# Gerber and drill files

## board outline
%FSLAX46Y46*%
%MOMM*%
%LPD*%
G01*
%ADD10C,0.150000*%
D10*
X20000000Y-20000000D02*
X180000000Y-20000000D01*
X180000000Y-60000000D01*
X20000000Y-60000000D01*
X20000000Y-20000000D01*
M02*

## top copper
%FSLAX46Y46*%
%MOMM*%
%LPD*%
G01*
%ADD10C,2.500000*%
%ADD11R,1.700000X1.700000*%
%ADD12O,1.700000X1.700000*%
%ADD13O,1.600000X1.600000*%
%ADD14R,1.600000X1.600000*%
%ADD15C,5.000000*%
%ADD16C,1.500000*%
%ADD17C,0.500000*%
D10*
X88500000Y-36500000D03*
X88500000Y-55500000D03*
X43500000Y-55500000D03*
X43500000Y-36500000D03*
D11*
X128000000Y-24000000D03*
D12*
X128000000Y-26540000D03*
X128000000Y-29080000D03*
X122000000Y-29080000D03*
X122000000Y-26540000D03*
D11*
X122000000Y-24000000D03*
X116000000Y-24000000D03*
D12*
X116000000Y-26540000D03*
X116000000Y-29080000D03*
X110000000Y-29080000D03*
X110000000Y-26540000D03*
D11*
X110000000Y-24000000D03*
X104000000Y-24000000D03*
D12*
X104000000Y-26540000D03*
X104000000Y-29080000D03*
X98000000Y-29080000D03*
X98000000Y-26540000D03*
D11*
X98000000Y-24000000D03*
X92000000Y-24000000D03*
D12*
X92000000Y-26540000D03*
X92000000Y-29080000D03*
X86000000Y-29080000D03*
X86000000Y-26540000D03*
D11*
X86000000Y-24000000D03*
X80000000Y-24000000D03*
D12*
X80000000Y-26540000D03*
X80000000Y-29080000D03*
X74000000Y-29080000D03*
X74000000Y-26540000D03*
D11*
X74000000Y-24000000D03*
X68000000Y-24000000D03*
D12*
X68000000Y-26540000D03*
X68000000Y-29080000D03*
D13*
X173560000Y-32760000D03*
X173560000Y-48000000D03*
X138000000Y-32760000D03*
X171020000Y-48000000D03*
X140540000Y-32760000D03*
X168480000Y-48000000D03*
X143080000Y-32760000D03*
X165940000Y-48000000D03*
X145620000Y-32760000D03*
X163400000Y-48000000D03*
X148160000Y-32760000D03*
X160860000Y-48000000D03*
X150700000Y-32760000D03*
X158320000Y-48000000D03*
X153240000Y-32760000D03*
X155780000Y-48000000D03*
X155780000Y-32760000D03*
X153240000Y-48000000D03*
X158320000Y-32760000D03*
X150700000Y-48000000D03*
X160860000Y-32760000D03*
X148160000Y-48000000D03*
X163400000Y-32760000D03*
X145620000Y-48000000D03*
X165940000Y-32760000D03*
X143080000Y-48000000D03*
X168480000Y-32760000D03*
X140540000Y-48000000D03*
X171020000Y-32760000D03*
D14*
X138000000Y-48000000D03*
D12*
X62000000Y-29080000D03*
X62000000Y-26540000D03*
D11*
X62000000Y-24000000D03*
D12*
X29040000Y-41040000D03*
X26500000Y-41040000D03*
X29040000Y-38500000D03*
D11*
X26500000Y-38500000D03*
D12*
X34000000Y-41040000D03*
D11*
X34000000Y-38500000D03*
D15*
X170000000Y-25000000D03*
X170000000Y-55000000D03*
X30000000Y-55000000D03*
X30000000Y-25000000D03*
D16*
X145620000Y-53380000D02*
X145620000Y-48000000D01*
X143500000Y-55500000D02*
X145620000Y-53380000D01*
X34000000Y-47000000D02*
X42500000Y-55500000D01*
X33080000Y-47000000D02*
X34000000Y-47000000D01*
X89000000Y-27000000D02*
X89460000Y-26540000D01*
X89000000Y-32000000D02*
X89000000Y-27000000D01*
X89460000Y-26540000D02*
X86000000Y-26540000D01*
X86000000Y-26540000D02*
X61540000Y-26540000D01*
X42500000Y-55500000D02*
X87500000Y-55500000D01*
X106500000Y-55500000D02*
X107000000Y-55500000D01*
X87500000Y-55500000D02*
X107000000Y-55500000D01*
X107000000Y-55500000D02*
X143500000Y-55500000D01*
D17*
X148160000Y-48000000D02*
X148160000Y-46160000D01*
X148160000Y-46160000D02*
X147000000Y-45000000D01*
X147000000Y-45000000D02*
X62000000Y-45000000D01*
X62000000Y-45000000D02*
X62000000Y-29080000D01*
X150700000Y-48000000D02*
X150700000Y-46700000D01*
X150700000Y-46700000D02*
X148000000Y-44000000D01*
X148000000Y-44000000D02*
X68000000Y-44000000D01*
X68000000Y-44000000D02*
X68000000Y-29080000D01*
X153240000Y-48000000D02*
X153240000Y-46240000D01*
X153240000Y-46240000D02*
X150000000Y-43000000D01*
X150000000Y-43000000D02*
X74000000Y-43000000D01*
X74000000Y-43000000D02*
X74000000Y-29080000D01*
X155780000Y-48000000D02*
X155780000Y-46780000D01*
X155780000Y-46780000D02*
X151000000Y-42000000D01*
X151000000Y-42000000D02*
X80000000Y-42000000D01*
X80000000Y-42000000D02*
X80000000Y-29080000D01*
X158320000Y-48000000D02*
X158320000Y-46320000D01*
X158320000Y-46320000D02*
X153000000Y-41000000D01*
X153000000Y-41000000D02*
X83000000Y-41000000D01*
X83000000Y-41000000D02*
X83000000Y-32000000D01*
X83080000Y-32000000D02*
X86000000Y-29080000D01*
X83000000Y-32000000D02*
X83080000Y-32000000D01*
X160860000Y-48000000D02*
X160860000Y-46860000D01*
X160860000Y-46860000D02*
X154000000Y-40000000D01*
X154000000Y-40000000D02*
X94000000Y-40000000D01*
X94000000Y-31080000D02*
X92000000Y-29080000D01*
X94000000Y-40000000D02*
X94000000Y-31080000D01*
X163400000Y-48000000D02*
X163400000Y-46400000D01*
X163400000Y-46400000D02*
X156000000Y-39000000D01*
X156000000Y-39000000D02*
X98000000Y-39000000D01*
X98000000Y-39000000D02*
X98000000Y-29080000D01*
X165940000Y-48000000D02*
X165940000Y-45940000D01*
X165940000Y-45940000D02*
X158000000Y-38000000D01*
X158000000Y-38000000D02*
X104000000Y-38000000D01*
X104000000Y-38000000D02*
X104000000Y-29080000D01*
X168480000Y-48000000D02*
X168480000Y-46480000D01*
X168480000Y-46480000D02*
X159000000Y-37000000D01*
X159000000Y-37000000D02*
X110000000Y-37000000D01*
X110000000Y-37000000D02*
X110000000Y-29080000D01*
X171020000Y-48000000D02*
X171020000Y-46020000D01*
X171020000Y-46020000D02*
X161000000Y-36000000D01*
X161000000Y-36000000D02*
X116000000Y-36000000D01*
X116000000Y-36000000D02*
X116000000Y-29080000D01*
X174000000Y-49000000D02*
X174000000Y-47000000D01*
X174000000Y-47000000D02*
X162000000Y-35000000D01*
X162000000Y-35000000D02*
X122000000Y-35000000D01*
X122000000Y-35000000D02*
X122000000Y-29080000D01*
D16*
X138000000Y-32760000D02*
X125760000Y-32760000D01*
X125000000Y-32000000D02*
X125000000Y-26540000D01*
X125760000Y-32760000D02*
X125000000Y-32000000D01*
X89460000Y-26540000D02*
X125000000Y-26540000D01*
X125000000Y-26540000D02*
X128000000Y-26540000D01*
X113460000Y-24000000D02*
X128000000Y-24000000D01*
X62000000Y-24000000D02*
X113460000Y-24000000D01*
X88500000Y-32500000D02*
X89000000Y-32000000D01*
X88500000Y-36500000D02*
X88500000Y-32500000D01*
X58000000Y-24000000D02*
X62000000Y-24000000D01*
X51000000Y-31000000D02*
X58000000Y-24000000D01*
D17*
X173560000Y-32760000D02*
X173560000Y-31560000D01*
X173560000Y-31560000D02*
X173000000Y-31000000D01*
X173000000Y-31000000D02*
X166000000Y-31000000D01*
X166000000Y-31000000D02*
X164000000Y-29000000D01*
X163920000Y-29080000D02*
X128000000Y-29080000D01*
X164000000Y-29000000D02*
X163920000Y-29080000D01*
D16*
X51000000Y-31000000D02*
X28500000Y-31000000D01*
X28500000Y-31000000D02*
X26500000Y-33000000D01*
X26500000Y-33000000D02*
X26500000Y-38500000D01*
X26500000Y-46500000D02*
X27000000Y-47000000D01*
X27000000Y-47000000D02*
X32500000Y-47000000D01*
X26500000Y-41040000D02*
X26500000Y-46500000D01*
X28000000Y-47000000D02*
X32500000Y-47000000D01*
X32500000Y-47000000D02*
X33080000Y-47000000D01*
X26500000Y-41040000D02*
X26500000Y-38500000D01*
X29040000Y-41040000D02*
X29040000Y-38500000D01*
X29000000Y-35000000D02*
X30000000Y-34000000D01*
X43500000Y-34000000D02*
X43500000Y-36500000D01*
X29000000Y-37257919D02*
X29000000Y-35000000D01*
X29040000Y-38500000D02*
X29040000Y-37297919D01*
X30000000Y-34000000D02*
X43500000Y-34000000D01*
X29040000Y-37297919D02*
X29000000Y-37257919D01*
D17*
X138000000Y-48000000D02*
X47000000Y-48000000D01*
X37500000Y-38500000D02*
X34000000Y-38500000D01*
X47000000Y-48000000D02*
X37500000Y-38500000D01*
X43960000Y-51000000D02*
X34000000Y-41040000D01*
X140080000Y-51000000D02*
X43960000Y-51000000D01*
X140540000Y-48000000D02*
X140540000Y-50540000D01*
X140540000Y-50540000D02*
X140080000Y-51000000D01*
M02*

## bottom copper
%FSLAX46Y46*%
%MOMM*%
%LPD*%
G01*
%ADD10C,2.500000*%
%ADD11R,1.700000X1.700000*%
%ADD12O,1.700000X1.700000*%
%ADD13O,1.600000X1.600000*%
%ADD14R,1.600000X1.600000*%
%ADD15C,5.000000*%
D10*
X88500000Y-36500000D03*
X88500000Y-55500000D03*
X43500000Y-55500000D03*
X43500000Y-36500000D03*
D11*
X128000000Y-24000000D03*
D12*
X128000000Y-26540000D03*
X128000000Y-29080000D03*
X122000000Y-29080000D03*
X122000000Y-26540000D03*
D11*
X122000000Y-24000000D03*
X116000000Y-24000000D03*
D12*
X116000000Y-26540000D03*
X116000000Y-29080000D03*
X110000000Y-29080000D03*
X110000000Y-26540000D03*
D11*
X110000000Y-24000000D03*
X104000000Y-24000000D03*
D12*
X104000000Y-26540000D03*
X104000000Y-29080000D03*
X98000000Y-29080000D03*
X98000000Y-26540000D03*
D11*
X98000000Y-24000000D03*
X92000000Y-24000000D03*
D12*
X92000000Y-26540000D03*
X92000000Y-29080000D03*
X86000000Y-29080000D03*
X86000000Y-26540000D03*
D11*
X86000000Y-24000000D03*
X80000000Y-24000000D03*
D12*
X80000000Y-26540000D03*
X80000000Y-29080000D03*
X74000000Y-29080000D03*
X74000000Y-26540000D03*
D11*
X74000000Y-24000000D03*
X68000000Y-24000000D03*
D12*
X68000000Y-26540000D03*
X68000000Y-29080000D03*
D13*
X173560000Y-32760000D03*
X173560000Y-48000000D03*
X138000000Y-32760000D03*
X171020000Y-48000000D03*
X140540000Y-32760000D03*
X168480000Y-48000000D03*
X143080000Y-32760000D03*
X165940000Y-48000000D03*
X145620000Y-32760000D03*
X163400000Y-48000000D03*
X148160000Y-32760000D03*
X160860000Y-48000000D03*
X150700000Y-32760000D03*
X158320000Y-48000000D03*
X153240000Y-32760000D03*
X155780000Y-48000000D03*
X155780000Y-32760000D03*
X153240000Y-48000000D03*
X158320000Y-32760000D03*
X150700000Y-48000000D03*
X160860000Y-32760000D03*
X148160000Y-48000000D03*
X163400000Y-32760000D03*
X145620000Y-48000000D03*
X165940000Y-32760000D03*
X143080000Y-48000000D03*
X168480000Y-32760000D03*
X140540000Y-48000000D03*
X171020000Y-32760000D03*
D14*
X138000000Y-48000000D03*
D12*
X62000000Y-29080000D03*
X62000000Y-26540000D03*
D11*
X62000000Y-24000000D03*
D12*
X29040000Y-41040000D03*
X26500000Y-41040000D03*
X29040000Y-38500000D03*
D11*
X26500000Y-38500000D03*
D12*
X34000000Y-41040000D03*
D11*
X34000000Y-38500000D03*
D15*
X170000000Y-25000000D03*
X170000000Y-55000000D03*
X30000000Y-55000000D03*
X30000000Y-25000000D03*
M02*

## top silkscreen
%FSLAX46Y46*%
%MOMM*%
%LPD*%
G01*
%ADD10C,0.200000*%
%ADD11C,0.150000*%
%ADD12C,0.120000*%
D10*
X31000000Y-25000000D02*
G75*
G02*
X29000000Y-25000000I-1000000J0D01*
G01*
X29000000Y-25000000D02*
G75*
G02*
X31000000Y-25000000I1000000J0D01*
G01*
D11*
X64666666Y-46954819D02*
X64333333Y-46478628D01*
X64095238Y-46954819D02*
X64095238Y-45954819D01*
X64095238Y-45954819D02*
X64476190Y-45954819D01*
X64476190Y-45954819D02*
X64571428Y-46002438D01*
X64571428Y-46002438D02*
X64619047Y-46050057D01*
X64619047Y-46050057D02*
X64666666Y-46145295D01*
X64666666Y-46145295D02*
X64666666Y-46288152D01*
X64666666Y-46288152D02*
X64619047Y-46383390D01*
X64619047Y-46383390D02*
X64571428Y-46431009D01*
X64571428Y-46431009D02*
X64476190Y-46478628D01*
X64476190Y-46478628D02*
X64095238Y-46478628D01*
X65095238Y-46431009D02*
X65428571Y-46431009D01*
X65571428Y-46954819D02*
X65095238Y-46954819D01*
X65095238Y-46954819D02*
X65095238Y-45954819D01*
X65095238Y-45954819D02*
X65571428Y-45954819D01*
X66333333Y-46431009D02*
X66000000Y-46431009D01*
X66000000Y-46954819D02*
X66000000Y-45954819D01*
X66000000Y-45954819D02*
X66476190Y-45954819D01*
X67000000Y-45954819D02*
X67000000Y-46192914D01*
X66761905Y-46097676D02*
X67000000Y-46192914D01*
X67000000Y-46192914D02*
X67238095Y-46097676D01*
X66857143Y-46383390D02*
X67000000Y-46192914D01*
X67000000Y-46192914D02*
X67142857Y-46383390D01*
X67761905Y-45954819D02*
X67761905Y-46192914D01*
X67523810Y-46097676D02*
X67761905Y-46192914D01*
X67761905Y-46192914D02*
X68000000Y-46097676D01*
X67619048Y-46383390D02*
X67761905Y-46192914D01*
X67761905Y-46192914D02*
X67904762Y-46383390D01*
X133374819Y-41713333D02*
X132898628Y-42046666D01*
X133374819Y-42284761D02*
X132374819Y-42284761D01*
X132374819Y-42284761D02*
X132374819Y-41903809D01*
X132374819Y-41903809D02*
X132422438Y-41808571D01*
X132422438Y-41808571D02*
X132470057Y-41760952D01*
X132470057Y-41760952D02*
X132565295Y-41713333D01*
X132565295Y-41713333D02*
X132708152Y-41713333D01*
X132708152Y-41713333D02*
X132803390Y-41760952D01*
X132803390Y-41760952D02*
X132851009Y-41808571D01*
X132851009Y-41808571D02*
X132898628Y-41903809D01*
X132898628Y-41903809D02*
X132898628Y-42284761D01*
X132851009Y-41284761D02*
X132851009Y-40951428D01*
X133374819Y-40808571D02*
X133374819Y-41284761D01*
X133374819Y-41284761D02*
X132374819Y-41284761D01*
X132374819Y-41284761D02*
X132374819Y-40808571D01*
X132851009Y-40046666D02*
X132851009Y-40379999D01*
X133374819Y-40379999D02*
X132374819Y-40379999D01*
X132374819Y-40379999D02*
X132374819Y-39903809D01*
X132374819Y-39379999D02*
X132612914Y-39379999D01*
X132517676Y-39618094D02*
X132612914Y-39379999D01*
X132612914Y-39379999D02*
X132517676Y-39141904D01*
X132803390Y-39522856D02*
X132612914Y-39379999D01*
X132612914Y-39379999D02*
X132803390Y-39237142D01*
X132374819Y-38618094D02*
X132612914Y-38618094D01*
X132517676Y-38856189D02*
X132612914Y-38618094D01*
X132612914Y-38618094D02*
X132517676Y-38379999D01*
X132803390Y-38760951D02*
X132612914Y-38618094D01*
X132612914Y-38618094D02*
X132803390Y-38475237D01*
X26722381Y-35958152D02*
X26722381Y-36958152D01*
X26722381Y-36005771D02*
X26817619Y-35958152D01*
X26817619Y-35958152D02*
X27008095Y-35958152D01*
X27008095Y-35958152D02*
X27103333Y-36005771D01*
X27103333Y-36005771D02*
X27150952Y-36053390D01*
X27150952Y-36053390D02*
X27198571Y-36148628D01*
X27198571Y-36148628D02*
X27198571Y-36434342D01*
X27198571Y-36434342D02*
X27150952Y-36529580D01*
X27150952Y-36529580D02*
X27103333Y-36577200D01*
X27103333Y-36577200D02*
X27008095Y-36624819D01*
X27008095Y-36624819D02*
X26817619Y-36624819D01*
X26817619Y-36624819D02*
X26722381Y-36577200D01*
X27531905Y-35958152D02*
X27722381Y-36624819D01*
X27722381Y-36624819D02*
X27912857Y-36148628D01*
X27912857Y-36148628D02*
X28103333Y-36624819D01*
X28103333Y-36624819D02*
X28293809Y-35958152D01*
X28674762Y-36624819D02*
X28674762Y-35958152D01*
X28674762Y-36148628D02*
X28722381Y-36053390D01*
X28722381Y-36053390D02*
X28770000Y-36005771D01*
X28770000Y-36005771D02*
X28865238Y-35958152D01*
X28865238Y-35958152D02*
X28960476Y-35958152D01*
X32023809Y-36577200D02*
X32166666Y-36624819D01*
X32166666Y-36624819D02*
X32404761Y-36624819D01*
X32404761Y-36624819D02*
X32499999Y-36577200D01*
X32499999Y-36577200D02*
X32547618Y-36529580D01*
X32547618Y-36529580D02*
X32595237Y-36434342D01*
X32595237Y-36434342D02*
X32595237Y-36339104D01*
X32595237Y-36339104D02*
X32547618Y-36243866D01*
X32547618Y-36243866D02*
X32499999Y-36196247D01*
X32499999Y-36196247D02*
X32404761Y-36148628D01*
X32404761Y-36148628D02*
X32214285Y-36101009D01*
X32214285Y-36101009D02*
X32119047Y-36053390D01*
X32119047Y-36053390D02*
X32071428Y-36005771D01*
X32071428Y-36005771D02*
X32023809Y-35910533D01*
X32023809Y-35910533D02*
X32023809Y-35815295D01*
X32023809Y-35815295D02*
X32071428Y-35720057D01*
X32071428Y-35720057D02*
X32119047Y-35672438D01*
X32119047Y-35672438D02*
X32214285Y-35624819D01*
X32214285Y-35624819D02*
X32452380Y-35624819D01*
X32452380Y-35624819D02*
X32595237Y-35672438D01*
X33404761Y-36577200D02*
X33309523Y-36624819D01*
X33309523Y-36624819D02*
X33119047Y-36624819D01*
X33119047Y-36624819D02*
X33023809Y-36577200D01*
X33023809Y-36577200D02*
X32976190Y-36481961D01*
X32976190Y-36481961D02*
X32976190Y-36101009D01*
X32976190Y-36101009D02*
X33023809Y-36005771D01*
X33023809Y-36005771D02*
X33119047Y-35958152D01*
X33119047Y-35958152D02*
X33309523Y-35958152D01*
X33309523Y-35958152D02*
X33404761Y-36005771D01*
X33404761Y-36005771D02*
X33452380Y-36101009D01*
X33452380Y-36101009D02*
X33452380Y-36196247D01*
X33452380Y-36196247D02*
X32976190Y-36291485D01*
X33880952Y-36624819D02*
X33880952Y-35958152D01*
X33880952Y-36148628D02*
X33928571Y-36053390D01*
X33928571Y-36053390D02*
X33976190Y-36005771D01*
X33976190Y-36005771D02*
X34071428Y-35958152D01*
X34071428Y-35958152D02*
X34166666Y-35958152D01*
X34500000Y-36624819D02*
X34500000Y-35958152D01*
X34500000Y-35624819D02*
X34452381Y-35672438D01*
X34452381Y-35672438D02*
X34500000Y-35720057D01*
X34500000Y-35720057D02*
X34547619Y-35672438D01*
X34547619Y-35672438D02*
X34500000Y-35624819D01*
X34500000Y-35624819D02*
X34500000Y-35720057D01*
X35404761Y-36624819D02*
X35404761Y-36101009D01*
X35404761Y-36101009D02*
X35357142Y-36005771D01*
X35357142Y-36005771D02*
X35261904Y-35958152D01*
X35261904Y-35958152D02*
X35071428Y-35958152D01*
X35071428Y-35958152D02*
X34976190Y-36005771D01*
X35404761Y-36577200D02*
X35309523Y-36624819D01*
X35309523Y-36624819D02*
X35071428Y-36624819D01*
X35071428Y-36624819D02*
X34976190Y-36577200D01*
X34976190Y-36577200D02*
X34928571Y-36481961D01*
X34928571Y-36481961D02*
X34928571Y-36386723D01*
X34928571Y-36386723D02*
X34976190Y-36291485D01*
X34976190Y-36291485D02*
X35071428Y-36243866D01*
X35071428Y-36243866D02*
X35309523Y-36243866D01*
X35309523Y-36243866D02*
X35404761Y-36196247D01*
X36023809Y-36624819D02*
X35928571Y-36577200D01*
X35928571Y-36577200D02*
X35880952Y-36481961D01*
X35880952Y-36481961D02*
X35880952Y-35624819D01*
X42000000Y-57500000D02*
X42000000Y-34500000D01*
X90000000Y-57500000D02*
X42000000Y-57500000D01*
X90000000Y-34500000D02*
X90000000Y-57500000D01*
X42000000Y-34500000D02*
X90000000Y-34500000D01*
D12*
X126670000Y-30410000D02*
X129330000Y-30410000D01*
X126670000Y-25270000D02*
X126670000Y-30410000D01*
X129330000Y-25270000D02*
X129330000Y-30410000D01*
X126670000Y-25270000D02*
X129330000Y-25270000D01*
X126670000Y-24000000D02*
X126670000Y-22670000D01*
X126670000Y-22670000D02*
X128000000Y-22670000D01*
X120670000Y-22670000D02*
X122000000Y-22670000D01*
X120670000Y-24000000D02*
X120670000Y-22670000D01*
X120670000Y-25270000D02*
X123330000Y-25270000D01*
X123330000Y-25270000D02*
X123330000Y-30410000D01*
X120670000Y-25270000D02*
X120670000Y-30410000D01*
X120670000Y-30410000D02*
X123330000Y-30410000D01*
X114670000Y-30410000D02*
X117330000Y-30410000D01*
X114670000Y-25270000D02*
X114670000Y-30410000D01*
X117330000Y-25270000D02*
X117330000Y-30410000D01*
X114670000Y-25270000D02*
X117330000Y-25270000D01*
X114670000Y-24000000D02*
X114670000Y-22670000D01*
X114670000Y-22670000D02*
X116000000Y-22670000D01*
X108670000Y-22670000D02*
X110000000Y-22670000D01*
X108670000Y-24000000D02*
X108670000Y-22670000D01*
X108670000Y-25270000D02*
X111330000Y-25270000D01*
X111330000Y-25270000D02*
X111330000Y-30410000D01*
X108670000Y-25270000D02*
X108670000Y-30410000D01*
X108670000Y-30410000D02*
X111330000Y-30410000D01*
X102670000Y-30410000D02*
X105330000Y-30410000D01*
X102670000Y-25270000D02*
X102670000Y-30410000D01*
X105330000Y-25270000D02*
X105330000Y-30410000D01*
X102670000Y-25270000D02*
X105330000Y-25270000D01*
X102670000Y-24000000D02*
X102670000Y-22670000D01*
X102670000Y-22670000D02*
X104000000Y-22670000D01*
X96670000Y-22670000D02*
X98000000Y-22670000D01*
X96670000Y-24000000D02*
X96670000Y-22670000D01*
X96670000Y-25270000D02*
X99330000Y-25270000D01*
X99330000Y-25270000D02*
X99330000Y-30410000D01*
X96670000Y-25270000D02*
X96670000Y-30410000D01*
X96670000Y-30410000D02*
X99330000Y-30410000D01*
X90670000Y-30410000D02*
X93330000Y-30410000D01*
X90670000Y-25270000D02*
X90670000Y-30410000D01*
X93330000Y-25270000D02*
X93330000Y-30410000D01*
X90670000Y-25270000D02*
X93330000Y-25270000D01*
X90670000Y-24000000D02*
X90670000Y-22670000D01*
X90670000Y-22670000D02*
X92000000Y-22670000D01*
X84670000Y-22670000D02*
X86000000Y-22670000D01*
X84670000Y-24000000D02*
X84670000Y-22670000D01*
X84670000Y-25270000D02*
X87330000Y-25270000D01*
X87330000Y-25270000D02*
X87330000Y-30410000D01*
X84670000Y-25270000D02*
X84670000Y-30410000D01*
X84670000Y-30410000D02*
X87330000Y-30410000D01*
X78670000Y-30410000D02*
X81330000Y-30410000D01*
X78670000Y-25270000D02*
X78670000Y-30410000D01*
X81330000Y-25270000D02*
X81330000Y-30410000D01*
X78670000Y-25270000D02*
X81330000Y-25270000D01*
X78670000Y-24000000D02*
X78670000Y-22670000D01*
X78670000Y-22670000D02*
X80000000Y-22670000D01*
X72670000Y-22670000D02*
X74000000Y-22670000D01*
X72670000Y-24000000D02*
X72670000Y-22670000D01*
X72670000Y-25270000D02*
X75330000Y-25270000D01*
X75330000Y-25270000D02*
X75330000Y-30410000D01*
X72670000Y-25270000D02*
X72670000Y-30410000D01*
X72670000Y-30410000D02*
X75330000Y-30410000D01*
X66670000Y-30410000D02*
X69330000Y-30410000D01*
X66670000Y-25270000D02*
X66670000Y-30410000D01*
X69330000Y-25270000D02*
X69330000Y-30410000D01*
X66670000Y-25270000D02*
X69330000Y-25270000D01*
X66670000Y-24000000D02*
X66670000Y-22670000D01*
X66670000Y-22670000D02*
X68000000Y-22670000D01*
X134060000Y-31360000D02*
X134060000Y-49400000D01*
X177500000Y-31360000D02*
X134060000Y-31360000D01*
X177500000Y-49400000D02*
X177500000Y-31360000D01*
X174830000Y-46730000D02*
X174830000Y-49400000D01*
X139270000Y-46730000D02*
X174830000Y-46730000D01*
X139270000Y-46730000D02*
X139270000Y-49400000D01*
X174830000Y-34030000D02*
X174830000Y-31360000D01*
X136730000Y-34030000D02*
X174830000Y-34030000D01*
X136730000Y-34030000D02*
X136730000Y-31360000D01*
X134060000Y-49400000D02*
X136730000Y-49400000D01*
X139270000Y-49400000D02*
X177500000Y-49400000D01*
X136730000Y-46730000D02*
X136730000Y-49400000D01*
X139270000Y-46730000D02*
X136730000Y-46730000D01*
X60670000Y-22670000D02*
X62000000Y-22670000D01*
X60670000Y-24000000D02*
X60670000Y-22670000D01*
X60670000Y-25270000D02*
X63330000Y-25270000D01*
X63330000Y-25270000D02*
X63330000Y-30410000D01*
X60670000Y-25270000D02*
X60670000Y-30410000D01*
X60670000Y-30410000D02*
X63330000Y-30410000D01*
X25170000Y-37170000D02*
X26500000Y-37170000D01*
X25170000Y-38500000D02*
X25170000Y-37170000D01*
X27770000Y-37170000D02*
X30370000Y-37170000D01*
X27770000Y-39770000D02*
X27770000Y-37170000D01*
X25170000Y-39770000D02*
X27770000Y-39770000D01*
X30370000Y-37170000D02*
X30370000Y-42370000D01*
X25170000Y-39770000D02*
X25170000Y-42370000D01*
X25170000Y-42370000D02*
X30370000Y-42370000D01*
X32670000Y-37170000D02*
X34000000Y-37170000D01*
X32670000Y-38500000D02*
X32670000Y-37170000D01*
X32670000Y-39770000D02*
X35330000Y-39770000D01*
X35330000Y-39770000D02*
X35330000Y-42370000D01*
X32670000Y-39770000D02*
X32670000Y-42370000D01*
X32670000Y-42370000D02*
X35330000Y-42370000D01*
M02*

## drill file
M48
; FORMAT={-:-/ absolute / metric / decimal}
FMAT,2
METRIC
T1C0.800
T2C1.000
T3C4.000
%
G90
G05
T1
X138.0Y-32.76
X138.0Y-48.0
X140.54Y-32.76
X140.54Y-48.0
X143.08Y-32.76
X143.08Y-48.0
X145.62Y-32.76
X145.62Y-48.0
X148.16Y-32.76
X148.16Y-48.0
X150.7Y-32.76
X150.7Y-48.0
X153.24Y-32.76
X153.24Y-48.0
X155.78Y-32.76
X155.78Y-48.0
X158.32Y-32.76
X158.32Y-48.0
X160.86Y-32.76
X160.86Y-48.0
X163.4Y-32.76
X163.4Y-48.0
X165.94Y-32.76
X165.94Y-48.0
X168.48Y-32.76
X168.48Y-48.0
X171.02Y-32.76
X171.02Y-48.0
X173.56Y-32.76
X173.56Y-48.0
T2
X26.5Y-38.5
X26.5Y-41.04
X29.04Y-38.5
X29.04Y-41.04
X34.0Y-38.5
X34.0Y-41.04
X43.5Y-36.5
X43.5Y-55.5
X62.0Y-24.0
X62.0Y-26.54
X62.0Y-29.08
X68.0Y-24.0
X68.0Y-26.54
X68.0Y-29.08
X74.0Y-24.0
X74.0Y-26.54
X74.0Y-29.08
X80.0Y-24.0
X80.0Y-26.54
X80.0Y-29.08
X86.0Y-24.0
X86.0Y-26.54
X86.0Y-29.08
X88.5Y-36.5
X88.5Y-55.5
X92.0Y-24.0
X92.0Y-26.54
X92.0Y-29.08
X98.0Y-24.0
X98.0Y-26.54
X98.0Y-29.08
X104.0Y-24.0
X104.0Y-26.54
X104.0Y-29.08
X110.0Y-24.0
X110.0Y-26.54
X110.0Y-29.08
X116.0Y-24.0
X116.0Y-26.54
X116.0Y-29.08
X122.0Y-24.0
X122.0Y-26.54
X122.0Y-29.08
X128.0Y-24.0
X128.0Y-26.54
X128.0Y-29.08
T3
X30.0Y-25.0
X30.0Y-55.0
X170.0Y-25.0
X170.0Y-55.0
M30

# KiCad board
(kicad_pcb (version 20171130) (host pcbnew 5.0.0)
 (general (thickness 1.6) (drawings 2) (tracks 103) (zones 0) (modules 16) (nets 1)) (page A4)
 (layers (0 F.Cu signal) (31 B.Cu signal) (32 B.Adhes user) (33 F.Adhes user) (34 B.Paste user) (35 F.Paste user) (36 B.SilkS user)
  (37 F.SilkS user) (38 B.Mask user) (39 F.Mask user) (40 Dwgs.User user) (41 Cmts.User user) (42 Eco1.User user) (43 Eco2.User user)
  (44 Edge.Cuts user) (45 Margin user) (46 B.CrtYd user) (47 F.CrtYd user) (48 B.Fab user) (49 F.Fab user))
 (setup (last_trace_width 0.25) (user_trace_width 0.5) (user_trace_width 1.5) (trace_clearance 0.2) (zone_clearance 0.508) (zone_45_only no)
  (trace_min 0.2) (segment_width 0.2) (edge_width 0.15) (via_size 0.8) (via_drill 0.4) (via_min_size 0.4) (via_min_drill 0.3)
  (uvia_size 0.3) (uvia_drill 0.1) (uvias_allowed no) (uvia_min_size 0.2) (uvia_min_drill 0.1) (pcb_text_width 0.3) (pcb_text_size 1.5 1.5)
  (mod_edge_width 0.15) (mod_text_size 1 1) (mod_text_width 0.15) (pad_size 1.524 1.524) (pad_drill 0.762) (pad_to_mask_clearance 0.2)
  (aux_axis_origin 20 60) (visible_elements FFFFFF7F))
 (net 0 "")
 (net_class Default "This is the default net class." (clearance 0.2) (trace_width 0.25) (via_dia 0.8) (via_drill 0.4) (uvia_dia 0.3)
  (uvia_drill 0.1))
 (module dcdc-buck (layer F.Cu) (at 66 46)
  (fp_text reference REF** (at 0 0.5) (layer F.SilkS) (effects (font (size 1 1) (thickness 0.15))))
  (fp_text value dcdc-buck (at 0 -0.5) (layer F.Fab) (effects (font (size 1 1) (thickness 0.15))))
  (fp_line (start -24 11.5) (end -24 -11.5) (layer F.SilkS) (width 0.15))
  (fp_line (start 24 11.5) (end -24 11.5) (layer F.SilkS) (width 0.15))
  (fp_line (start 24 -11.5) (end 24 11.5) (layer F.SilkS) (width 0.15))
  (fp_line (start -24 -11.5) (end 24 -11.5) (layer F.SilkS) (width 0.15))
  (pad 4 thru_hole circle (at 22.5 -9.5) (size 2.5 2.5) (drill 1) (layers *.Cu *.Mask))
  (pad 3 thru_hole circle (at 22.5 9.5) (size 2.5 2.5) (drill 1) (layers *.Cu *.Mask))
  (pad 2 thru_hole circle (at -22.5 9.5) (size 2.5 2.5) (drill 1) (layers *.Cu *.Mask))
  (pad 1 thru_hole circle (at -22.5 -9.5) (size 2.5 2.5) (drill 1) (layers *.Cu *.Mask)))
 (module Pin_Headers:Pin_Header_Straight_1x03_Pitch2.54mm (layer F.Cu) (at 128 24)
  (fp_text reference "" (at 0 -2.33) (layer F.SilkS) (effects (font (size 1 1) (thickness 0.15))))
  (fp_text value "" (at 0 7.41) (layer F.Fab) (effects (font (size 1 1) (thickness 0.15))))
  (fp_line (start -1.33 6.41) (end 1.33 6.41) (layer F.SilkS) (width 0.12))
  (fp_line (start -1.33 1.27) (end -1.33 6.41) (layer F.SilkS) (width 0.12))
  (fp_line (start 1.33 1.27) (end 1.33 6.41) (layer F.SilkS) (width 0.12))
  (fp_line (start -1.33 1.27) (end 1.33 1.27) (layer F.SilkS) (width 0.12))
  (fp_line (start -1.33 0) (end -1.33 -1.33) (layer F.SilkS) (width 0.12))
  (fp_line (start -1.33 -1.33) (end 0 -1.33) (layer F.SilkS) (width 0.12))
  (pad 1 thru_hole rect (at 0 0) (size 1.7 1.7) (drill 1) (layers *.Cu *.Mask))
  (pad 2 thru_hole oval (at 0 2.54) (size 1.7 1.7) (drill 1) (layers *.Cu *.Mask))
  (pad 3 thru_hole oval (at 0 5.08) (size 1.7 1.7) (drill 1) (layers *.Cu *.Mask)))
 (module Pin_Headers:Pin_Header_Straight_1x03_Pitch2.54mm (layer F.Cu) (at 122 24)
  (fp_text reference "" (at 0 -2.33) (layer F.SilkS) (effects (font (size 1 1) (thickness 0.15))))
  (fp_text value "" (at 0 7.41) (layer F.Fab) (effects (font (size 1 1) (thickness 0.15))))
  (fp_line (start -1.33 -1.33) (end 0 -1.33) (layer F.SilkS) (width 0.12))
  (fp_line (start -1.33 0) (end -1.33 -1.33) (layer F.SilkS) (width 0.12))
  (fp_line (start -1.33 1.27) (end 1.33 1.27) (layer F.SilkS) (width 0.12))
  (fp_line (start 1.33 1.27) (end 1.33 6.41) (layer F.SilkS) (width 0.12))
  (fp_line (start -1.33 1.27) (end -1.33 6.41) (layer F.SilkS) (width 0.12))
  (fp_line (start -1.33 6.41) (end 1.33 6.41) (layer F.SilkS) (width 0.12))
  (pad 3 thru_hole oval (at 0 5.08) (size 1.7 1.7) (drill 1) (layers *.Cu *.Mask))
  (pad 2 thru_hole oval (at 0 2.54) (size 1.7 1.7) (drill 1) (layers *.Cu *.Mask))
  (pad 1 thru_hole rect (at 0 0) (size 1.7 1.7) (drill 1) (layers *.Cu *.Mask)))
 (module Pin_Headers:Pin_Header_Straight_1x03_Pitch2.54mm (layer F.Cu) (at 116 24)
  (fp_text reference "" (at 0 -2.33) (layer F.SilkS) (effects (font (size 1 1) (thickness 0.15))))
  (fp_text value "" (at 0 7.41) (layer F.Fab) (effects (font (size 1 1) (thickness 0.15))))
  (fp_line (start -1.33 6.41) (end 1.33 6.41) (layer F.SilkS) (width 0.12))
  (fp_line (start -1.33 1.27) (end -1.33 6.41) (layer F.SilkS) (width 0.12))
  (fp_line (start 1.33 1.27) (end 1.33 6.41) (layer F.SilkS) (width 0.12))
  (fp_line (start -1.33 1.27) (end 1.33 1.27) (layer F.SilkS) (width 0.12))
  (fp_line (start -1.33 0) (end -1.33 -1.33) (layer F.SilkS) (width 0.12))
  (fp_line (start -1.33 -1.33) (end 0 -1.33) (layer F.SilkS) (width 0.12))
  (pad 1 thru_hole rect (at 0 0) (size 1.7 1.7) (drill 1) (layers *.Cu *.Mask))
  (pad 2 thru_hole oval (at 0 2.54) (size 1.7 1.7) (drill 1) (layers *.Cu *.Mask))
  (pad 3 thru_hole oval (at 0 5.08) (size 1.7 1.7) (drill 1) (layers *.Cu *.Mask)))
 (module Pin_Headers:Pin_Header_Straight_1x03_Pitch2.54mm (layer F.Cu) (at 110 24)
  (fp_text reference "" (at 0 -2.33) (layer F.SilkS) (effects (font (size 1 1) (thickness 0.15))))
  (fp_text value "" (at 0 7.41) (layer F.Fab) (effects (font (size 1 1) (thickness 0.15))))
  (fp_line (start -1.33 -1.33) (end 0 -1.33) (layer F.SilkS) (width 0.12))
  (fp_line (start -1.33 0) (end -1.33 -1.33) (layer F.SilkS) (width 0.12))
  (fp_line (start -1.33 1.27) (end 1.33 1.27) (layer F.SilkS) (width 0.12))
  (fp_line (start 1.33 1.27) (end 1.33 6.41) (layer F.SilkS) (width 0.12))
  (fp_line (start -1.33 1.27) (end -1.33 6.41) (layer F.SilkS) (width 0.12))
  (fp_line (start -1.33 6.41) (end 1.33 6.41) (layer F.SilkS) (width 0.12))
  (pad 3 thru_hole oval (at 0 5.08) (size 1.7 1.7) (drill 1) (layers *.Cu *.Mask))
  (pad 2 thru_hole oval (at 0 2.54) (size 1.7 1.7) (drill 1) (layers *.Cu *.Mask))
  (pad 1 thru_hole rect (at 0 0) (size 1.7 1.7) (drill 1) (layers *.Cu *.Mask)))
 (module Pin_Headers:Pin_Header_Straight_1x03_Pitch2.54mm (layer F.Cu) (at 104 24)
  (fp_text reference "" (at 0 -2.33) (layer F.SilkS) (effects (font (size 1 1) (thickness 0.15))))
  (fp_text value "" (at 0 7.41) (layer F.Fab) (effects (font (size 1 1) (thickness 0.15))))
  (fp_line (start -1.33 6.41) (end 1.33 6.41) (layer F.SilkS) (width 0.12))
  (fp_line (start -1.33 1.27) (end -1.33 6.41) (layer F.SilkS) (width 0.12))
  (fp_line (start 1.33 1.27) (end 1.33 6.41) (layer F.SilkS) (width 0.12))
  (fp_line (start -1.33 1.27) (end 1.33 1.27) (layer F.SilkS) (width 0.12))
  (fp_line (start -1.33 0) (end -1.33 -1.33) (layer F.SilkS) (width 0.12))
  (fp_line (start -1.33 -1.33) (end 0 -1.33) (layer F.SilkS) (width 0.12))
  (pad 1 thru_hole rect (at 0 0) (size 1.7 1.7) (drill 1) (layers *.Cu *.Mask))
  (pad 2 thru_hole oval (at 0 2.54) (size 1.7 1.7) (drill 1) (layers *.Cu *.Mask))
  (pad 3 thru_hole oval (at 0 5.08) (size 1.7 1.7) (drill 1) (layers *.Cu *.Mask)))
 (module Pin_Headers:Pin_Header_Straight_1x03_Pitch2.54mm (layer F.Cu) (at 98 24)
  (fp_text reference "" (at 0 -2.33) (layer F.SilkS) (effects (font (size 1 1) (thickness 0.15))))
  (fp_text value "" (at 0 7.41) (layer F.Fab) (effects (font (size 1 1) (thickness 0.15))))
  (fp_line (start -1.33 -1.33) (end 0 -1.33) (layer F.SilkS) (width 0.12))
  (fp_line (start -1.33 0) (end -1.33 -1.33) (layer F.SilkS) (width 0.12))
  (fp_line (start -1.33 1.27) (end 1.33 1.27) (layer F.SilkS) (width 0.12))
  (fp_line (start 1.33 1.27) (end 1.33 6.41) (layer F.SilkS) (width 0.12))
  (fp_line (start -1.33 1.27) (end -1.33 6.41) (layer F.SilkS) (width 0.12))
  (fp_line (start -1.33 6.41) (end 1.33 6.41) (layer F.SilkS) (width 0.12))
  (pad 3 thru_hole oval (at 0 5.08) (size 1.7 1.7) (drill 1) (layers *.Cu *.Mask))
  (pad 2 thru_hole oval (at 0 2.54) (size 1.7 1.7) (drill 1) (layers *.Cu *.Mask))
  (pad 1 thru_hole rect (at 0 0) (size 1.7 1.7) (drill 1) (layers *.Cu *.Mask)))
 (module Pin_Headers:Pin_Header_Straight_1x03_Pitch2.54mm (layer F.Cu) (at 92 24)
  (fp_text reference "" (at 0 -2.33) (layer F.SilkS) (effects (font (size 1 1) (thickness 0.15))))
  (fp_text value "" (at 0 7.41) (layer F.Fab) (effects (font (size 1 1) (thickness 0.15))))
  (fp_line (start -1.33 6.41) (end 1.33 6.41) (layer F.SilkS) (width 0.12))
  (fp_line (start -1.33 1.27) (end -1.33 6.41) (layer F.SilkS) (width 0.12))
  (fp_line (start 1.33 1.27) (end 1.33 6.41) (layer F.SilkS) (width 0.12))
  (fp_line (start -1.33 1.27) (end 1.33 1.27) (layer F.SilkS) (width 0.12))
  (fp_line (start -1.33 0) (end -1.33 -1.33) (layer F.SilkS) (width 0.12))
  (fp_line (start -1.33 -1.33) (end 0 -1.33) (layer F.SilkS) (width 0.12))
  (pad 1 thru_hole rect (at 0 0) (size 1.7 1.7) (drill 1) (layers *.Cu *.Mask))
  (pad 2 thru_hole oval (at 0 2.54) (size 1.7 1.7) (drill 1) (layers *.Cu *.Mask))
  (pad 3 thru_hole oval (at 0 5.08) (size 1.7 1.7) (drill 1) (layers *.Cu *.Mask)))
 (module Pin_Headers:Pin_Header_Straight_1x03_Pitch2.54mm (layer F.Cu) (at 86 24)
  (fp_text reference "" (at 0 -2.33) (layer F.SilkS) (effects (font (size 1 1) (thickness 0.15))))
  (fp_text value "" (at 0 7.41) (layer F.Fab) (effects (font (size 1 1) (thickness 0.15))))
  (fp_line (start -1.33 -1.33) (end 0 -1.33) (layer F.SilkS) (width 0.12))
  (fp_line (start -1.33 0) (end -1.33 -1.33) (layer F.SilkS) (width 0.12))
  (fp_line (start -1.33 1.27) (end 1.33 1.27) (layer F.SilkS) (width 0.12))
  (fp_line (start 1.33 1.27) (end 1.33 6.41) (layer F.SilkS) (width 0.12))
  (fp_line (start -1.33 1.27) (end -1.33 6.41) (layer F.SilkS) (width 0.12))
  (fp_line (start -1.33 6.41) (end 1.33 6.41) (layer F.SilkS) (width 0.12))
  (pad 3 thru_hole oval (at 0 5.08) (size 1.7 1.7) (drill 1) (layers *.Cu *.Mask))
  (pad 2 thru_hole oval (at 0 2.54) (size 1.7 1.7) (drill 1) (layers *.Cu *.Mask))
  (pad 1 thru_hole rect (at 0 0) (size 1.7 1.7) (drill 1) (layers *.Cu *.Mask)))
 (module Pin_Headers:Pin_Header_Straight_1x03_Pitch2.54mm (layer F.Cu) (at 80 24)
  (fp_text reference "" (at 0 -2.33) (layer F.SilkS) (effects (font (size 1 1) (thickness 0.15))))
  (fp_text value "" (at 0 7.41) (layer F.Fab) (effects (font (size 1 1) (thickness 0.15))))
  (fp_line (start -1.33 6.41) (end 1.33 6.41) (layer F.SilkS) (width 0.12))
  (fp_line (start -1.33 1.27) (end -1.33 6.41) (layer F.SilkS) (width 0.12))
  (fp_line (start 1.33 1.27) (end 1.33 6.41) (layer F.SilkS) (width 0.12))
  (fp_line (start -1.33 1.27) (end 1.33 1.27) (layer F.SilkS) (width 0.12))
  (fp_line (start -1.33 0) (end -1.33 -1.33) (layer F.SilkS) (width 0.12))
  (fp_line (start -1.33 -1.33) (end 0 -1.33) (layer F.SilkS) (width 0.12))
  (pad 1 thru_hole rect (at 0 0) (size 1.7 1.7) (drill 1) (layers *.Cu *.Mask))
  (pad 2 thru_hole oval (at 0 2.54) (size 1.7 1.7) (drill 1) (layers *.Cu *.Mask))
  (pad 3 thru_hole oval (at 0 5.08) (size 1.7 1.7) (drill 1) (layers *.Cu *.Mask)))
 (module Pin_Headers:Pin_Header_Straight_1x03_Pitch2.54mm (layer F.Cu) (at 74 24)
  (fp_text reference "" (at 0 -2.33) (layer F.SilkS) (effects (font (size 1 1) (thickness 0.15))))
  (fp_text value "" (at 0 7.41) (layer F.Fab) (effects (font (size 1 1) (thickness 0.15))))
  (fp_line (start -1.33 -1.33) (end 0 -1.33) (layer F.SilkS) (width 0.12))
  (fp_line (start -1.33 0) (end -1.33 -1.33) (layer F.SilkS) (width 0.12))
  (fp_line (start -1.33 1.27) (end 1.33 1.27) (layer F.SilkS) (width 0.12))
  (fp_line (start 1.33 1.27) (end 1.33 6.41) (layer F.SilkS) (width 0.12))
  (fp_line (start -1.33 1.27) (end -1.33 6.41) (layer F.SilkS) (width 0.12))
  (fp_line (start -1.33 6.41) (end 1.33 6.41) (layer F.SilkS) (width 0.12))
  (pad 3 thru_hole oval (at 0 5.08) (size 1.7 1.7) (drill 1) (layers *.Cu *.Mask))
  (pad 2 thru_hole oval (at 0 2.54) (size 1.7 1.7) (drill 1) (layers *.Cu *.Mask))
  (pad 1 thru_hole rect (at 0 0) (size 1.7 1.7) (drill 1) (layers *.Cu *.Mask)))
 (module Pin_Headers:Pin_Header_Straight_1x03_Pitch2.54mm (layer F.Cu) (at 68 24)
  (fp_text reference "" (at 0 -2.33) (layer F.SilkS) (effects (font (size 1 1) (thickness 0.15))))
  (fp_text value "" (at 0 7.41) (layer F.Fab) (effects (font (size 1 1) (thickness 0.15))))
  (fp_line (start -1.33 6.41) (end 1.33 6.41) (layer F.SilkS) (width 0.12))
  (fp_line (start -1.33 1.27) (end -1.33 6.41) (layer F.SilkS) (width 0.12))
  (fp_line (start 1.33 1.27) (end 1.33 6.41) (layer F.SilkS) (width 0.12))
  (fp_line (start -1.33 1.27) (end 1.33 1.27) (layer F.SilkS) (width 0.12))
  (fp_line (start -1.33 0) (end -1.33 -1.33) (layer F.SilkS) (width 0.12))
  (fp_line (start -1.33 -1.33) (end 0 -1.33) (layer F.SilkS) (width 0.12))
  (pad 1 thru_hole rect (at 0 0) (size 1.7 1.7) (drill 1) (layers *.Cu *.Mask))
  (pad 2 thru_hole oval (at 0 2.54) (size 1.7 1.7) (drill 1) (layers *.Cu *.Mask))
  (pad 3 thru_hole oval (at 0 5.08) (size 1.7 1.7) (drill 1) (layers *.Cu *.Mask)))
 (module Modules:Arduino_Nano (layer F.Cu) (at 138 48 90)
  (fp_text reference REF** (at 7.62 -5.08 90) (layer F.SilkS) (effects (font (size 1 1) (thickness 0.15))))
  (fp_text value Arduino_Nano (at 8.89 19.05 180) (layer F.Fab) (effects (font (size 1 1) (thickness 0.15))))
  (fp_line (start 16.64 -3.94) (end -1.4 -3.94) (layer F.SilkS) (width 0.12))
  (fp_line (start 16.64 39.5) (end 16.64 -3.94) (layer F.SilkS) (width 0.12))
  (fp_line (start -1.4 39.5) (end 16.64 39.5) (layer F.SilkS) (width 0.12))
  (fp_line (start 1.27 36.83) (end -1.4 36.83) (layer F.SilkS) (width 0.12))
  (fp_line (start 1.27 1.27) (end 1.27 36.83) (layer F.SilkS) (width 0.12))
  (fp_line (start 1.27 1.27) (end -1.4 1.27) (layer F.SilkS) (width 0.12))
  (fp_line (start 13.97 36.83) (end 16.64 36.83) (layer F.SilkS) (width 0.12))
  (fp_line (start 13.97 -1.27) (end 13.97 36.83) (layer F.SilkS) (width 0.12))
  (fp_line (start 13.97 -1.27) (end 16.64 -1.27) (layer F.SilkS) (width 0.12))
  (fp_line (start -1.4 -3.94) (end -1.4 -1.27) (layer F.SilkS) (width 0.12))
  (fp_line (start -1.4 1.27) (end -1.4 39.5) (layer F.SilkS) (width 0.12))
  (fp_line (start 1.27 -1.27) (end -1.4 -1.27) (layer F.SilkS) (width 0.12))
  (fp_line (start 1.27 1.27) (end 1.27 -1.27) (layer F.SilkS) (width 0.12))
  (pad 16 thru_hole oval (at 15.24 35.56 90) (size 1.6 1.6) (drill 0.8) (layers *.Cu *.Mask))
  (pad 15 thru_hole oval (at 0 35.56 90) (size 1.6 1.6) (drill 0.8) (layers *.Cu *.Mask))
  (pad 30 thru_hole oval (at 15.24 0 90) (size 1.6 1.6) (drill 0.8) (layers *.Cu *.Mask))
  (pad 14 thru_hole oval (at 0 33.02 90) (size 1.6 1.6) (drill 0.8) (layers *.Cu *.Mask))
  (pad 29 thru_hole oval (at 15.24 2.54 90) (size 1.6 1.6) (drill 0.8) (layers *.Cu *.Mask))
  (pad 13 thru_hole oval (at 0 30.48 90) (size 1.6 1.6) (drill 0.8) (layers *.Cu *.Mask))
  (pad 28 thru_hole oval (at 15.24 5.08 90) (size 1.6 1.6) (drill 0.8) (layers *.Cu *.Mask))
  (pad 12 thru_hole oval (at 0 27.94 90) (size 1.6 1.6) (drill 0.8) (layers *.Cu *.Mask))
  (pad 27 thru_hole oval (at 15.24 7.62 90) (size 1.6 1.6) (drill 0.8) (layers *.Cu *.Mask))
  (pad 11 thru_hole oval (at 0 25.4 90) (size 1.6 1.6) (drill 0.8) (layers *.Cu *.Mask))
  (pad 26 thru_hole oval (at 15.24 10.16 90) (size 1.6 1.6) (drill 0.8) (layers *.Cu *.Mask))
  (pad 10 thru_hole oval (at 0 22.86 90) (size 1.6 1.6) (drill 0.8) (layers *.Cu *.Mask))
  (pad 25 thru_hole oval (at 15.24 12.7 90) (size 1.6 1.6) (drill 0.8) (layers *.Cu *.Mask))
  (pad 9 thru_hole oval (at 0 20.32 90) (size 1.6 1.6) (drill 0.8) (layers *.Cu *.Mask))
  (pad 24 thru_hole oval (at 15.24 15.24 90) (size 1.6 1.6) (drill 0.8) (layers *.Cu *.Mask))
  (pad 8 thru_hole oval (at 0 17.78 90) (size 1.6 1.6) (drill 0.8) (layers *.Cu *.Mask))
  (pad 23 thru_hole oval (at 15.24 17.78 90) (size 1.6 1.6) (drill 0.8) (layers *.Cu *.Mask))
  (pad 7 thru_hole oval (at 0 15.24 90) (size 1.6 1.6) (drill 0.8) (layers *.Cu *.Mask))
  (pad 22 thru_hole oval (at 15.24 20.32 90) (size 1.6 1.6) (drill 0.8) (layers *.Cu *.Mask))
  (pad 6 thru_hole oval (at 0 12.7 90) (size 1.6 1.6) (drill 0.8) (layers *.Cu *.Mask))
  (pad 21 thru_hole oval (at 15.24 22.86 90) (size 1.6 1.6) (drill 0.8) (layers *.Cu *.Mask))
  (pad 5 thru_hole oval (at 0 10.16 90) (size 1.6 1.6) (drill 0.8) (layers *.Cu *.Mask))
  (pad 20 thru_hole oval (at 15.24 25.4 90) (size 1.6 1.6) (drill 0.8) (layers *.Cu *.Mask))
  (pad 4 thru_hole oval (at 0 7.62 90) (size 1.6 1.6) (drill 0.8) (layers *.Cu *.Mask))
  (pad 19 thru_hole oval (at 15.24 27.94 90) (size 1.6 1.6) (drill 0.8) (layers *.Cu *.Mask))
  (pad 3 thru_hole oval (at 0 5.08 90) (size 1.6 1.6) (drill 0.8) (layers *.Cu *.Mask))
  (pad 18 thru_hole oval (at 15.24 30.48 90) (size 1.6 1.6) (drill 0.8) (layers *.Cu *.Mask))
  (pad 2 thru_hole oval (at 0 2.54 90) (size 1.6 1.6) (drill 0.8) (layers *.Cu *.Mask))
  (pad 17 thru_hole oval (at 15.24 33.02 90) (size 1.6 1.6) (drill 0.8) (layers *.Cu *.Mask))
  (pad 1 thru_hole rect (at 0 0 90) (size 1.6 1.6) (drill 0.8) (layers *.Cu *.Mask)))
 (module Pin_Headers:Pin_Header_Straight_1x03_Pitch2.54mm (layer F.Cu) (at 62 24)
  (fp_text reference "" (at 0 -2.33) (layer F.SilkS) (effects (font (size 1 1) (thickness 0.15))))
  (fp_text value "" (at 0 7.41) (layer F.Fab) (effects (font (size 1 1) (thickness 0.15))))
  (fp_line (start -1.33 -1.33) (end 0 -1.33) (layer F.SilkS) (width 0.12))
  (fp_line (start -1.33 0) (end -1.33 -1.33) (layer F.SilkS) (width 0.12))
  (fp_line (start -1.33 1.27) (end 1.33 1.27) (layer F.SilkS) (width 0.12))
  (fp_line (start 1.33 1.27) (end 1.33 6.41) (layer F.SilkS) (width 0.12))
  (fp_line (start -1.33 1.27) (end -1.33 6.41) (layer F.SilkS) (width 0.12))
  (fp_line (start -1.33 6.41) (end 1.33 6.41) (layer F.SilkS) (width 0.12))
  (pad 3 thru_hole oval (at 0 5.08) (size 1.7 1.7) (drill 1) (layers *.Cu *.Mask))
  (pad 2 thru_hole oval (at 0 2.54) (size 1.7 1.7) (drill 1) (layers *.Cu *.Mask))
  (pad 1 thru_hole rect (at 0 0) (size 1.7 1.7) (drill 1) (layers *.Cu *.Mask)))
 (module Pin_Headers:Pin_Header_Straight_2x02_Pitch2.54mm (layer F.Cu) (at 26.5 38.5)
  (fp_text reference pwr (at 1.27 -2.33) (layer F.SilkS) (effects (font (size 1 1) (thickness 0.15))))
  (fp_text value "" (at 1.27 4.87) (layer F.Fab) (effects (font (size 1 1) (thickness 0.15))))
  (fp_line (start -1.33 -1.33) (end 0 -1.33) (layer F.SilkS) (width 0.12))
  (fp_line (start -1.33 0) (end -1.33 -1.33) (layer F.SilkS) (width 0.12))
  (fp_line (start 1.27 -1.33) (end 3.87 -1.33) (layer F.SilkS) (width 0.12))
  (fp_line (start 1.27 1.27) (end 1.27 -1.33) (layer F.SilkS) (width 0.12))
  (fp_line (start -1.33 1.27) (end 1.27 1.27) (layer F.SilkS) (width 0.12))
  (fp_line (start 3.87 -1.33) (end 3.87 3.87) (layer F.SilkS) (width 0.12))
  (fp_line (start -1.33 1.27) (end -1.33 3.87) (layer F.SilkS) (width 0.12))
  (fp_line (start -1.33 3.87) (end 3.87 3.87) (layer F.SilkS) (width 0.12))
  (pad 4 thru_hole oval (at 2.54 2.54) (size 1.7 1.7) (drill 1) (layers *.Cu *.Mask))
  (pad 3 thru_hole oval (at 0 2.54) (size 1.7 1.7) (drill 1) (layers *.Cu *.Mask))
  (pad 2 thru_hole oval (at 2.54 0) (size 1.7 1.7) (drill 1) (layers *.Cu *.Mask))
  (pad 1 thru_hole rect (at 0 0) (size 1.7 1.7) (drill 1) (layers *.Cu *.Mask)))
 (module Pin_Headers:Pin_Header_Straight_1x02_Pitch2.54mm (layer F.Cu) (at 34 38.5)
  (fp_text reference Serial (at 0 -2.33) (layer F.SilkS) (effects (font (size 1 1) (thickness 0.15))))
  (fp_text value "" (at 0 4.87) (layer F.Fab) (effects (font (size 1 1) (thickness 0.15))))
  (fp_line (start -1.33 -1.33) (end 0 -1.33) (layer F.SilkS) (width 0.12))
  (fp_line (start -1.33 0) (end -1.33 -1.33) (layer F.SilkS) (width 0.12))
  (fp_line (start -1.33 1.27) (end 1.33 1.27) (layer F.SilkS) (width 0.12))
  (fp_line (start 1.33 1.27) (end 1.33 3.87) (layer F.SilkS) (width 0.12))
  (fp_line (start -1.33 1.27) (end -1.33 3.87) (layer F.SilkS) (width 0.12))
  (fp_line (start -1.33 3.87) (end 1.33 3.87) (layer F.SilkS) (width 0.12))
  (pad 2 thru_hole oval (at 0 2.54) (size 1.7 1.7) (drill 1) (layers *.Cu *.Mask))
  (pad 1 thru_hole rect (at 0 0) (size 1.7 1.7) (drill 1) (layers *.Cu *.Mask)))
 (gr_circle (center 30 25) (end 30 26) (layer F.SilkS) (width 0.2))
 (gr_poly (pts (xy 20 20) (xy 180 20) (xy 180 60) (xy 20 60)) (layer Edge.Cuts) (width 0.15))
 (segment (start 145.62 53.38) (end 145.62 48) (width 1.5) (layer F.Cu) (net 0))
 (segment (start 143.5 55.5) (end 145.62 53.38) (width 1.5) (layer F.Cu) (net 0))
 (segment (start 34 47) (end 42.5 55.5) (width 1.5) (layer F.Cu) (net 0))
 (segment (start 33.08 47) (end 34 47) (width 1.5) (layer F.Cu) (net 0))
 (segment (start 89 27) (end 89.46 26.54) (width 1.5) (layer F.Cu) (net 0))
 (segment (start 89 32) (end 89 27) (width 1.5) (layer F.Cu) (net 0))
 (segment (start 89.46 26.54) (end 86 26.54) (width 1.5) (layer F.Cu) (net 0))
 (segment (start 86 26.54) (end 61.54 26.54) (width 1.5) (layer F.Cu) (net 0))
 (segment (start 42.5 55.5) (end 87.5 55.5) (width 1.5) (layer F.Cu) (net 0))
 (segment (start 106.5 55.5) (end 107 55.5) (width 1.5) (layer F.Cu) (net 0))
 (segment (start 87.5 55.5) (end 107 55.5) (width 1.5) (layer F.Cu) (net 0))
 (segment (start 107 55.5) (end 143.5 55.5) (width 1.5) (layer F.Cu) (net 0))
 (segment (start 148.16 48) (end 148.16 46.16) (width 0.5) (layer F.Cu) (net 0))
 (segment (start 148.16 46.16) (end 147 45) (width 0.5) (layer F.Cu) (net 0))
 (segment (start 147 45) (end 62 45) (width 0.5) (layer F.Cu) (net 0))
 (segment (start 62 45) (end 62 29.08) (width 0.5) (layer F.Cu) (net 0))
 (segment (start 150.7 48) (end 150.7 46.7) (width 0.5) (layer F.Cu) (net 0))
 (segment (start 150.7 46.7) (end 148 44) (width 0.5) (layer F.Cu) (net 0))
 (segment (start 148 44) (end 68 44) (width 0.5) (layer F.Cu) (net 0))
 (segment (start 68 44) (end 68 29.08) (width 0.5) (layer F.Cu) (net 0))
 (segment (start 153.24 48) (end 153.24 46.24) (width 0.5) (layer F.Cu) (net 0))
 (segment (start 153.24 46.24) (end 150 43) (width 0.5) (layer F.Cu) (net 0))
 (segment (start 150 43) (end 74 43) (width 0.5) (layer F.Cu) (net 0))
 (segment (start 74 43) (end 74 29.08) (width 0.5) (layer F.Cu) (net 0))
 (segment (start 155.78 48) (end 155.78 46.78) (width 0.5) (layer F.Cu) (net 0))
 (segment (start 155.78 46.78) (end 151 42) (width 0.5) (layer F.Cu) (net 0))
 (segment (start 151 42) (end 80 42) (width 0.5) (layer F.Cu) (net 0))
 (segment (start 80 42) (end 80 29.08) (width 0.5) (layer F.Cu) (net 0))
 (segment (start 158.32 48) (end 158.32 46.32) (width 0.5) (layer F.Cu) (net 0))
 (segment (start 158.32 46.32) (end 153 41) (width 0.5) (layer F.Cu) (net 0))
 (segment (start 153 41) (end 83 41) (width 0.5) (layer F.Cu) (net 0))
 (segment (start 83 41) (end 83 32) (width 0.5) (layer F.Cu) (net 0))
 (segment (start 83.08 32) (end 86 29.08) (width 0.5) (layer F.Cu) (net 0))
 (segment (start 83 32) (end 83.08 32) (width 0.5) (layer F.Cu) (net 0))
 (segment (start 160.86 48) (end 160.86 46.86) (width 0.5) (layer F.Cu) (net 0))
 (segment (start 160.86 46.86) (end 154 40) (width 0.5) (layer F.Cu) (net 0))
 (segment (start 154 40) (end 94 40) (width 0.5) (layer F.Cu) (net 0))
 (segment (start 94 31.08) (end 92 29.08) (width 0.5) (layer F.Cu) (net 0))
 (segment (start 94 40) (end 94 31.08) (width 0.5) (layer F.Cu) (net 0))
 (segment (start 163.4 48) (end 163.4 46.4) (width 0.5) (layer F.Cu) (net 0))
 (segment (start 163.4 46.4) (end 156 39) (width 0.5) (layer F.Cu) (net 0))
 (segment (start 156 39) (end 98 39) (width 0.5) (layer F.Cu) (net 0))
 (segment (start 98 39) (end 98 29.08) (width 0.5) (layer F.Cu) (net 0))
 (segment (start 165.94 48) (end 165.94 45.94) (width 0.5) (layer F.Cu) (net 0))
 (segment (start 165.94 45.94) (end 158 38) (width 0.5) (layer F.Cu) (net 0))
 (segment (start 158 38) (end 104 38) (width 0.5) (layer F.Cu) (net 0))
 (segment (start 104 38) (end 104 29.08) (width 0.5) (layer F.Cu) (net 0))
 (segment (start 168.48 48) (end 168.48 46.48) (width 0.5) (layer F.Cu) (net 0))
 (segment (start 168.48 46.48) (end 159 37) (width 0.5) (layer F.Cu) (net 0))
 (segment (start 159 37) (end 110 37) (width 0.5) (layer F.Cu) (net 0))
 (segment (start 110 37) (end 110 29.08) (width 0.5) (layer F.Cu) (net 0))
 (segment (start 171.02 48) (end 171.02 46.02) (width 0.5) (layer F.Cu) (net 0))
 (segment (start 171.02 46.02) (end 161 36) (width 0.5) (layer F.Cu) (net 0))
 (segment (start 161 36) (end 116 36) (width 0.5) (layer F.Cu) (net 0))
 (segment (start 116 36) (end 116 29.08) (width 0.5) (layer F.Cu) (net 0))
 (segment (start 174 49) (end 174 47) (width 0.5) (layer F.Cu) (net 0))
 (segment (start 174 47) (end 162 35) (width 0.5) (layer F.Cu) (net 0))
 (segment (start 162 35) (end 122 35) (width 0.5) (layer F.Cu) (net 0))
 (segment (start 122 35) (end 122 29.08) (width 0.5) (layer F.Cu) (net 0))
 (segment (start 138 32.76) (end 125.76 32.76) (width 1.5) (layer F.Cu) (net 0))
 (segment (start 125 32) (end 125 26.54) (width 1.5) (layer F.Cu) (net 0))
 (segment (start 125.76 32.76) (end 125 32) (width 1.5) (layer F.Cu) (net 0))
 (segment (start 89.46 26.54) (end 125 26.54) (width 1.5) (layer F.Cu) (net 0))
 (segment (start 125 26.54) (end 128 26.54) (width 1.5) (layer F.Cu) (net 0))
 (segment (start 113.46 24) (end 128 24) (width 1.5) (layer F.Cu) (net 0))
 (segment (start 62 24) (end 113.46 24) (width 1.5) (layer F.Cu) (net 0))
 (segment (start 88.5 32.5) (end 89 32) (width 1.5) (layer F.Cu) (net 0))
 (segment (start 88.5 36.5) (end 88.5 32.5) (width 1.5) (layer F.Cu) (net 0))
 (via (at 170 25) (size 5) (drill 4) (layers F.Cu B.Cu) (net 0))
 (via (at 170 55) (size 5) (drill 4) (layers F.Cu B.Cu) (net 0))
 (via (at 30 55) (size 5) (drill 4) (layers F.Cu B.Cu) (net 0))
 (via (at 30 25) (size 5) (drill 4) (layers F.Cu B.Cu) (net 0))
 (segment (start 58 24) (end 62 24) (width 1.5) (layer F.Cu) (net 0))
 (segment (start 51 31) (end 58 24) (width 1.5) (layer F.Cu) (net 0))
 (segment (start 173.56 32.76) (end 173.56 31.56) (width 0.5) (layer F.Cu) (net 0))
 (segment (start 173.56 31.56) (end 173 31) (width 0.5) (layer F.Cu) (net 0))
 (segment (start 173 31) (end 166 31) (width 0.5) (layer F.Cu) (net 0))
 (segment (start 166 31) (end 164 29) (width 0.5) (layer F.Cu) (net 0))
 (segment (start 163.92 29.08) (end 128 29.08) (width 0.5) (layer F.Cu) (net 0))
 (segment (start 164 29) (end 163.92 29.08) (width 0.5) (layer F.Cu) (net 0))
 (segment (start 51 31) (end 28.5 31) (width 1.5) (layer F.Cu) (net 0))
 (segment (start 28.5 31) (end 26.5 33) (width 1.5) (layer F.Cu) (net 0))
 (segment (start 26.5 33) (end 26.5 38.5) (width 1.5) (layer F.Cu) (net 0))
 (segment (start 26.5 46.5) (end 27 47) (width 1.5) (layer F.Cu) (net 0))
 (segment (start 27 47) (end 32.5 47) (width 1.5) (layer F.Cu) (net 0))
 (segment (start 26.5 41.04) (end 26.5 46.5) (width 1.5) (layer F.Cu) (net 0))
 (segment (start 28 47) (end 32.5 47) (width 1.5) (layer F.Cu) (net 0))
 (segment (start 32.5 47) (end 33.08 47) (width 1.5) (layer F.Cu) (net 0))
 (segment (start 26.5 41.04) (end 26.5 38.5) (width 1.5) (layer F.Cu) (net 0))
 (segment (start 29.04 41.04) (end 29.04 38.5) (width 1.5) (layer F.Cu) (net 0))
 (segment (start 29 35) (end 30 34) (width 1.5) (layer F.Cu) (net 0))
 (segment (start 43.5 34) (end 43.5 36.5) (width 1.5) (layer F.Cu) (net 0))
 (segment (start 29 37.257919) (end 29 35) (width 1.5) (layer F.Cu) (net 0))
 (segment (start 29.04 38.5) (end 29.04 37.297919) (width 1.5) (layer F.Cu) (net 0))
 (segment (start 30 34) (end 43.5 34) (width 1.5) (layer F.Cu) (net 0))
 (segment (start 29.04 37.297919) (end 29 37.257919) (width 1.5) (layer F.Cu) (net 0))
 (segment (start 138 48) (end 47 48) (width 0.5) (layer F.Cu) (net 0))
 (segment (start 37.5 38.5) (end 34 38.5) (width 0.5) (layer F.Cu) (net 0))
 (segment (start 47 48) (end 37.5 38.5) (width 0.5) (layer F.Cu) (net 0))
 (segment (start 43.96 51) (end 34 41.04) (width 0.5) (layer F.Cu) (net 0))
 (segment (start 140.08 51) (end 43.96 51) (width 0.5) (layer F.Cu) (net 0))
 (segment (start 140.54 48) (end 140.54 50.54) (width 0.5) (layer F.Cu) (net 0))
 (segment (start 140.54 50.54) (end 140.08 51) (width 0.5) (layer F.Cu) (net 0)))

